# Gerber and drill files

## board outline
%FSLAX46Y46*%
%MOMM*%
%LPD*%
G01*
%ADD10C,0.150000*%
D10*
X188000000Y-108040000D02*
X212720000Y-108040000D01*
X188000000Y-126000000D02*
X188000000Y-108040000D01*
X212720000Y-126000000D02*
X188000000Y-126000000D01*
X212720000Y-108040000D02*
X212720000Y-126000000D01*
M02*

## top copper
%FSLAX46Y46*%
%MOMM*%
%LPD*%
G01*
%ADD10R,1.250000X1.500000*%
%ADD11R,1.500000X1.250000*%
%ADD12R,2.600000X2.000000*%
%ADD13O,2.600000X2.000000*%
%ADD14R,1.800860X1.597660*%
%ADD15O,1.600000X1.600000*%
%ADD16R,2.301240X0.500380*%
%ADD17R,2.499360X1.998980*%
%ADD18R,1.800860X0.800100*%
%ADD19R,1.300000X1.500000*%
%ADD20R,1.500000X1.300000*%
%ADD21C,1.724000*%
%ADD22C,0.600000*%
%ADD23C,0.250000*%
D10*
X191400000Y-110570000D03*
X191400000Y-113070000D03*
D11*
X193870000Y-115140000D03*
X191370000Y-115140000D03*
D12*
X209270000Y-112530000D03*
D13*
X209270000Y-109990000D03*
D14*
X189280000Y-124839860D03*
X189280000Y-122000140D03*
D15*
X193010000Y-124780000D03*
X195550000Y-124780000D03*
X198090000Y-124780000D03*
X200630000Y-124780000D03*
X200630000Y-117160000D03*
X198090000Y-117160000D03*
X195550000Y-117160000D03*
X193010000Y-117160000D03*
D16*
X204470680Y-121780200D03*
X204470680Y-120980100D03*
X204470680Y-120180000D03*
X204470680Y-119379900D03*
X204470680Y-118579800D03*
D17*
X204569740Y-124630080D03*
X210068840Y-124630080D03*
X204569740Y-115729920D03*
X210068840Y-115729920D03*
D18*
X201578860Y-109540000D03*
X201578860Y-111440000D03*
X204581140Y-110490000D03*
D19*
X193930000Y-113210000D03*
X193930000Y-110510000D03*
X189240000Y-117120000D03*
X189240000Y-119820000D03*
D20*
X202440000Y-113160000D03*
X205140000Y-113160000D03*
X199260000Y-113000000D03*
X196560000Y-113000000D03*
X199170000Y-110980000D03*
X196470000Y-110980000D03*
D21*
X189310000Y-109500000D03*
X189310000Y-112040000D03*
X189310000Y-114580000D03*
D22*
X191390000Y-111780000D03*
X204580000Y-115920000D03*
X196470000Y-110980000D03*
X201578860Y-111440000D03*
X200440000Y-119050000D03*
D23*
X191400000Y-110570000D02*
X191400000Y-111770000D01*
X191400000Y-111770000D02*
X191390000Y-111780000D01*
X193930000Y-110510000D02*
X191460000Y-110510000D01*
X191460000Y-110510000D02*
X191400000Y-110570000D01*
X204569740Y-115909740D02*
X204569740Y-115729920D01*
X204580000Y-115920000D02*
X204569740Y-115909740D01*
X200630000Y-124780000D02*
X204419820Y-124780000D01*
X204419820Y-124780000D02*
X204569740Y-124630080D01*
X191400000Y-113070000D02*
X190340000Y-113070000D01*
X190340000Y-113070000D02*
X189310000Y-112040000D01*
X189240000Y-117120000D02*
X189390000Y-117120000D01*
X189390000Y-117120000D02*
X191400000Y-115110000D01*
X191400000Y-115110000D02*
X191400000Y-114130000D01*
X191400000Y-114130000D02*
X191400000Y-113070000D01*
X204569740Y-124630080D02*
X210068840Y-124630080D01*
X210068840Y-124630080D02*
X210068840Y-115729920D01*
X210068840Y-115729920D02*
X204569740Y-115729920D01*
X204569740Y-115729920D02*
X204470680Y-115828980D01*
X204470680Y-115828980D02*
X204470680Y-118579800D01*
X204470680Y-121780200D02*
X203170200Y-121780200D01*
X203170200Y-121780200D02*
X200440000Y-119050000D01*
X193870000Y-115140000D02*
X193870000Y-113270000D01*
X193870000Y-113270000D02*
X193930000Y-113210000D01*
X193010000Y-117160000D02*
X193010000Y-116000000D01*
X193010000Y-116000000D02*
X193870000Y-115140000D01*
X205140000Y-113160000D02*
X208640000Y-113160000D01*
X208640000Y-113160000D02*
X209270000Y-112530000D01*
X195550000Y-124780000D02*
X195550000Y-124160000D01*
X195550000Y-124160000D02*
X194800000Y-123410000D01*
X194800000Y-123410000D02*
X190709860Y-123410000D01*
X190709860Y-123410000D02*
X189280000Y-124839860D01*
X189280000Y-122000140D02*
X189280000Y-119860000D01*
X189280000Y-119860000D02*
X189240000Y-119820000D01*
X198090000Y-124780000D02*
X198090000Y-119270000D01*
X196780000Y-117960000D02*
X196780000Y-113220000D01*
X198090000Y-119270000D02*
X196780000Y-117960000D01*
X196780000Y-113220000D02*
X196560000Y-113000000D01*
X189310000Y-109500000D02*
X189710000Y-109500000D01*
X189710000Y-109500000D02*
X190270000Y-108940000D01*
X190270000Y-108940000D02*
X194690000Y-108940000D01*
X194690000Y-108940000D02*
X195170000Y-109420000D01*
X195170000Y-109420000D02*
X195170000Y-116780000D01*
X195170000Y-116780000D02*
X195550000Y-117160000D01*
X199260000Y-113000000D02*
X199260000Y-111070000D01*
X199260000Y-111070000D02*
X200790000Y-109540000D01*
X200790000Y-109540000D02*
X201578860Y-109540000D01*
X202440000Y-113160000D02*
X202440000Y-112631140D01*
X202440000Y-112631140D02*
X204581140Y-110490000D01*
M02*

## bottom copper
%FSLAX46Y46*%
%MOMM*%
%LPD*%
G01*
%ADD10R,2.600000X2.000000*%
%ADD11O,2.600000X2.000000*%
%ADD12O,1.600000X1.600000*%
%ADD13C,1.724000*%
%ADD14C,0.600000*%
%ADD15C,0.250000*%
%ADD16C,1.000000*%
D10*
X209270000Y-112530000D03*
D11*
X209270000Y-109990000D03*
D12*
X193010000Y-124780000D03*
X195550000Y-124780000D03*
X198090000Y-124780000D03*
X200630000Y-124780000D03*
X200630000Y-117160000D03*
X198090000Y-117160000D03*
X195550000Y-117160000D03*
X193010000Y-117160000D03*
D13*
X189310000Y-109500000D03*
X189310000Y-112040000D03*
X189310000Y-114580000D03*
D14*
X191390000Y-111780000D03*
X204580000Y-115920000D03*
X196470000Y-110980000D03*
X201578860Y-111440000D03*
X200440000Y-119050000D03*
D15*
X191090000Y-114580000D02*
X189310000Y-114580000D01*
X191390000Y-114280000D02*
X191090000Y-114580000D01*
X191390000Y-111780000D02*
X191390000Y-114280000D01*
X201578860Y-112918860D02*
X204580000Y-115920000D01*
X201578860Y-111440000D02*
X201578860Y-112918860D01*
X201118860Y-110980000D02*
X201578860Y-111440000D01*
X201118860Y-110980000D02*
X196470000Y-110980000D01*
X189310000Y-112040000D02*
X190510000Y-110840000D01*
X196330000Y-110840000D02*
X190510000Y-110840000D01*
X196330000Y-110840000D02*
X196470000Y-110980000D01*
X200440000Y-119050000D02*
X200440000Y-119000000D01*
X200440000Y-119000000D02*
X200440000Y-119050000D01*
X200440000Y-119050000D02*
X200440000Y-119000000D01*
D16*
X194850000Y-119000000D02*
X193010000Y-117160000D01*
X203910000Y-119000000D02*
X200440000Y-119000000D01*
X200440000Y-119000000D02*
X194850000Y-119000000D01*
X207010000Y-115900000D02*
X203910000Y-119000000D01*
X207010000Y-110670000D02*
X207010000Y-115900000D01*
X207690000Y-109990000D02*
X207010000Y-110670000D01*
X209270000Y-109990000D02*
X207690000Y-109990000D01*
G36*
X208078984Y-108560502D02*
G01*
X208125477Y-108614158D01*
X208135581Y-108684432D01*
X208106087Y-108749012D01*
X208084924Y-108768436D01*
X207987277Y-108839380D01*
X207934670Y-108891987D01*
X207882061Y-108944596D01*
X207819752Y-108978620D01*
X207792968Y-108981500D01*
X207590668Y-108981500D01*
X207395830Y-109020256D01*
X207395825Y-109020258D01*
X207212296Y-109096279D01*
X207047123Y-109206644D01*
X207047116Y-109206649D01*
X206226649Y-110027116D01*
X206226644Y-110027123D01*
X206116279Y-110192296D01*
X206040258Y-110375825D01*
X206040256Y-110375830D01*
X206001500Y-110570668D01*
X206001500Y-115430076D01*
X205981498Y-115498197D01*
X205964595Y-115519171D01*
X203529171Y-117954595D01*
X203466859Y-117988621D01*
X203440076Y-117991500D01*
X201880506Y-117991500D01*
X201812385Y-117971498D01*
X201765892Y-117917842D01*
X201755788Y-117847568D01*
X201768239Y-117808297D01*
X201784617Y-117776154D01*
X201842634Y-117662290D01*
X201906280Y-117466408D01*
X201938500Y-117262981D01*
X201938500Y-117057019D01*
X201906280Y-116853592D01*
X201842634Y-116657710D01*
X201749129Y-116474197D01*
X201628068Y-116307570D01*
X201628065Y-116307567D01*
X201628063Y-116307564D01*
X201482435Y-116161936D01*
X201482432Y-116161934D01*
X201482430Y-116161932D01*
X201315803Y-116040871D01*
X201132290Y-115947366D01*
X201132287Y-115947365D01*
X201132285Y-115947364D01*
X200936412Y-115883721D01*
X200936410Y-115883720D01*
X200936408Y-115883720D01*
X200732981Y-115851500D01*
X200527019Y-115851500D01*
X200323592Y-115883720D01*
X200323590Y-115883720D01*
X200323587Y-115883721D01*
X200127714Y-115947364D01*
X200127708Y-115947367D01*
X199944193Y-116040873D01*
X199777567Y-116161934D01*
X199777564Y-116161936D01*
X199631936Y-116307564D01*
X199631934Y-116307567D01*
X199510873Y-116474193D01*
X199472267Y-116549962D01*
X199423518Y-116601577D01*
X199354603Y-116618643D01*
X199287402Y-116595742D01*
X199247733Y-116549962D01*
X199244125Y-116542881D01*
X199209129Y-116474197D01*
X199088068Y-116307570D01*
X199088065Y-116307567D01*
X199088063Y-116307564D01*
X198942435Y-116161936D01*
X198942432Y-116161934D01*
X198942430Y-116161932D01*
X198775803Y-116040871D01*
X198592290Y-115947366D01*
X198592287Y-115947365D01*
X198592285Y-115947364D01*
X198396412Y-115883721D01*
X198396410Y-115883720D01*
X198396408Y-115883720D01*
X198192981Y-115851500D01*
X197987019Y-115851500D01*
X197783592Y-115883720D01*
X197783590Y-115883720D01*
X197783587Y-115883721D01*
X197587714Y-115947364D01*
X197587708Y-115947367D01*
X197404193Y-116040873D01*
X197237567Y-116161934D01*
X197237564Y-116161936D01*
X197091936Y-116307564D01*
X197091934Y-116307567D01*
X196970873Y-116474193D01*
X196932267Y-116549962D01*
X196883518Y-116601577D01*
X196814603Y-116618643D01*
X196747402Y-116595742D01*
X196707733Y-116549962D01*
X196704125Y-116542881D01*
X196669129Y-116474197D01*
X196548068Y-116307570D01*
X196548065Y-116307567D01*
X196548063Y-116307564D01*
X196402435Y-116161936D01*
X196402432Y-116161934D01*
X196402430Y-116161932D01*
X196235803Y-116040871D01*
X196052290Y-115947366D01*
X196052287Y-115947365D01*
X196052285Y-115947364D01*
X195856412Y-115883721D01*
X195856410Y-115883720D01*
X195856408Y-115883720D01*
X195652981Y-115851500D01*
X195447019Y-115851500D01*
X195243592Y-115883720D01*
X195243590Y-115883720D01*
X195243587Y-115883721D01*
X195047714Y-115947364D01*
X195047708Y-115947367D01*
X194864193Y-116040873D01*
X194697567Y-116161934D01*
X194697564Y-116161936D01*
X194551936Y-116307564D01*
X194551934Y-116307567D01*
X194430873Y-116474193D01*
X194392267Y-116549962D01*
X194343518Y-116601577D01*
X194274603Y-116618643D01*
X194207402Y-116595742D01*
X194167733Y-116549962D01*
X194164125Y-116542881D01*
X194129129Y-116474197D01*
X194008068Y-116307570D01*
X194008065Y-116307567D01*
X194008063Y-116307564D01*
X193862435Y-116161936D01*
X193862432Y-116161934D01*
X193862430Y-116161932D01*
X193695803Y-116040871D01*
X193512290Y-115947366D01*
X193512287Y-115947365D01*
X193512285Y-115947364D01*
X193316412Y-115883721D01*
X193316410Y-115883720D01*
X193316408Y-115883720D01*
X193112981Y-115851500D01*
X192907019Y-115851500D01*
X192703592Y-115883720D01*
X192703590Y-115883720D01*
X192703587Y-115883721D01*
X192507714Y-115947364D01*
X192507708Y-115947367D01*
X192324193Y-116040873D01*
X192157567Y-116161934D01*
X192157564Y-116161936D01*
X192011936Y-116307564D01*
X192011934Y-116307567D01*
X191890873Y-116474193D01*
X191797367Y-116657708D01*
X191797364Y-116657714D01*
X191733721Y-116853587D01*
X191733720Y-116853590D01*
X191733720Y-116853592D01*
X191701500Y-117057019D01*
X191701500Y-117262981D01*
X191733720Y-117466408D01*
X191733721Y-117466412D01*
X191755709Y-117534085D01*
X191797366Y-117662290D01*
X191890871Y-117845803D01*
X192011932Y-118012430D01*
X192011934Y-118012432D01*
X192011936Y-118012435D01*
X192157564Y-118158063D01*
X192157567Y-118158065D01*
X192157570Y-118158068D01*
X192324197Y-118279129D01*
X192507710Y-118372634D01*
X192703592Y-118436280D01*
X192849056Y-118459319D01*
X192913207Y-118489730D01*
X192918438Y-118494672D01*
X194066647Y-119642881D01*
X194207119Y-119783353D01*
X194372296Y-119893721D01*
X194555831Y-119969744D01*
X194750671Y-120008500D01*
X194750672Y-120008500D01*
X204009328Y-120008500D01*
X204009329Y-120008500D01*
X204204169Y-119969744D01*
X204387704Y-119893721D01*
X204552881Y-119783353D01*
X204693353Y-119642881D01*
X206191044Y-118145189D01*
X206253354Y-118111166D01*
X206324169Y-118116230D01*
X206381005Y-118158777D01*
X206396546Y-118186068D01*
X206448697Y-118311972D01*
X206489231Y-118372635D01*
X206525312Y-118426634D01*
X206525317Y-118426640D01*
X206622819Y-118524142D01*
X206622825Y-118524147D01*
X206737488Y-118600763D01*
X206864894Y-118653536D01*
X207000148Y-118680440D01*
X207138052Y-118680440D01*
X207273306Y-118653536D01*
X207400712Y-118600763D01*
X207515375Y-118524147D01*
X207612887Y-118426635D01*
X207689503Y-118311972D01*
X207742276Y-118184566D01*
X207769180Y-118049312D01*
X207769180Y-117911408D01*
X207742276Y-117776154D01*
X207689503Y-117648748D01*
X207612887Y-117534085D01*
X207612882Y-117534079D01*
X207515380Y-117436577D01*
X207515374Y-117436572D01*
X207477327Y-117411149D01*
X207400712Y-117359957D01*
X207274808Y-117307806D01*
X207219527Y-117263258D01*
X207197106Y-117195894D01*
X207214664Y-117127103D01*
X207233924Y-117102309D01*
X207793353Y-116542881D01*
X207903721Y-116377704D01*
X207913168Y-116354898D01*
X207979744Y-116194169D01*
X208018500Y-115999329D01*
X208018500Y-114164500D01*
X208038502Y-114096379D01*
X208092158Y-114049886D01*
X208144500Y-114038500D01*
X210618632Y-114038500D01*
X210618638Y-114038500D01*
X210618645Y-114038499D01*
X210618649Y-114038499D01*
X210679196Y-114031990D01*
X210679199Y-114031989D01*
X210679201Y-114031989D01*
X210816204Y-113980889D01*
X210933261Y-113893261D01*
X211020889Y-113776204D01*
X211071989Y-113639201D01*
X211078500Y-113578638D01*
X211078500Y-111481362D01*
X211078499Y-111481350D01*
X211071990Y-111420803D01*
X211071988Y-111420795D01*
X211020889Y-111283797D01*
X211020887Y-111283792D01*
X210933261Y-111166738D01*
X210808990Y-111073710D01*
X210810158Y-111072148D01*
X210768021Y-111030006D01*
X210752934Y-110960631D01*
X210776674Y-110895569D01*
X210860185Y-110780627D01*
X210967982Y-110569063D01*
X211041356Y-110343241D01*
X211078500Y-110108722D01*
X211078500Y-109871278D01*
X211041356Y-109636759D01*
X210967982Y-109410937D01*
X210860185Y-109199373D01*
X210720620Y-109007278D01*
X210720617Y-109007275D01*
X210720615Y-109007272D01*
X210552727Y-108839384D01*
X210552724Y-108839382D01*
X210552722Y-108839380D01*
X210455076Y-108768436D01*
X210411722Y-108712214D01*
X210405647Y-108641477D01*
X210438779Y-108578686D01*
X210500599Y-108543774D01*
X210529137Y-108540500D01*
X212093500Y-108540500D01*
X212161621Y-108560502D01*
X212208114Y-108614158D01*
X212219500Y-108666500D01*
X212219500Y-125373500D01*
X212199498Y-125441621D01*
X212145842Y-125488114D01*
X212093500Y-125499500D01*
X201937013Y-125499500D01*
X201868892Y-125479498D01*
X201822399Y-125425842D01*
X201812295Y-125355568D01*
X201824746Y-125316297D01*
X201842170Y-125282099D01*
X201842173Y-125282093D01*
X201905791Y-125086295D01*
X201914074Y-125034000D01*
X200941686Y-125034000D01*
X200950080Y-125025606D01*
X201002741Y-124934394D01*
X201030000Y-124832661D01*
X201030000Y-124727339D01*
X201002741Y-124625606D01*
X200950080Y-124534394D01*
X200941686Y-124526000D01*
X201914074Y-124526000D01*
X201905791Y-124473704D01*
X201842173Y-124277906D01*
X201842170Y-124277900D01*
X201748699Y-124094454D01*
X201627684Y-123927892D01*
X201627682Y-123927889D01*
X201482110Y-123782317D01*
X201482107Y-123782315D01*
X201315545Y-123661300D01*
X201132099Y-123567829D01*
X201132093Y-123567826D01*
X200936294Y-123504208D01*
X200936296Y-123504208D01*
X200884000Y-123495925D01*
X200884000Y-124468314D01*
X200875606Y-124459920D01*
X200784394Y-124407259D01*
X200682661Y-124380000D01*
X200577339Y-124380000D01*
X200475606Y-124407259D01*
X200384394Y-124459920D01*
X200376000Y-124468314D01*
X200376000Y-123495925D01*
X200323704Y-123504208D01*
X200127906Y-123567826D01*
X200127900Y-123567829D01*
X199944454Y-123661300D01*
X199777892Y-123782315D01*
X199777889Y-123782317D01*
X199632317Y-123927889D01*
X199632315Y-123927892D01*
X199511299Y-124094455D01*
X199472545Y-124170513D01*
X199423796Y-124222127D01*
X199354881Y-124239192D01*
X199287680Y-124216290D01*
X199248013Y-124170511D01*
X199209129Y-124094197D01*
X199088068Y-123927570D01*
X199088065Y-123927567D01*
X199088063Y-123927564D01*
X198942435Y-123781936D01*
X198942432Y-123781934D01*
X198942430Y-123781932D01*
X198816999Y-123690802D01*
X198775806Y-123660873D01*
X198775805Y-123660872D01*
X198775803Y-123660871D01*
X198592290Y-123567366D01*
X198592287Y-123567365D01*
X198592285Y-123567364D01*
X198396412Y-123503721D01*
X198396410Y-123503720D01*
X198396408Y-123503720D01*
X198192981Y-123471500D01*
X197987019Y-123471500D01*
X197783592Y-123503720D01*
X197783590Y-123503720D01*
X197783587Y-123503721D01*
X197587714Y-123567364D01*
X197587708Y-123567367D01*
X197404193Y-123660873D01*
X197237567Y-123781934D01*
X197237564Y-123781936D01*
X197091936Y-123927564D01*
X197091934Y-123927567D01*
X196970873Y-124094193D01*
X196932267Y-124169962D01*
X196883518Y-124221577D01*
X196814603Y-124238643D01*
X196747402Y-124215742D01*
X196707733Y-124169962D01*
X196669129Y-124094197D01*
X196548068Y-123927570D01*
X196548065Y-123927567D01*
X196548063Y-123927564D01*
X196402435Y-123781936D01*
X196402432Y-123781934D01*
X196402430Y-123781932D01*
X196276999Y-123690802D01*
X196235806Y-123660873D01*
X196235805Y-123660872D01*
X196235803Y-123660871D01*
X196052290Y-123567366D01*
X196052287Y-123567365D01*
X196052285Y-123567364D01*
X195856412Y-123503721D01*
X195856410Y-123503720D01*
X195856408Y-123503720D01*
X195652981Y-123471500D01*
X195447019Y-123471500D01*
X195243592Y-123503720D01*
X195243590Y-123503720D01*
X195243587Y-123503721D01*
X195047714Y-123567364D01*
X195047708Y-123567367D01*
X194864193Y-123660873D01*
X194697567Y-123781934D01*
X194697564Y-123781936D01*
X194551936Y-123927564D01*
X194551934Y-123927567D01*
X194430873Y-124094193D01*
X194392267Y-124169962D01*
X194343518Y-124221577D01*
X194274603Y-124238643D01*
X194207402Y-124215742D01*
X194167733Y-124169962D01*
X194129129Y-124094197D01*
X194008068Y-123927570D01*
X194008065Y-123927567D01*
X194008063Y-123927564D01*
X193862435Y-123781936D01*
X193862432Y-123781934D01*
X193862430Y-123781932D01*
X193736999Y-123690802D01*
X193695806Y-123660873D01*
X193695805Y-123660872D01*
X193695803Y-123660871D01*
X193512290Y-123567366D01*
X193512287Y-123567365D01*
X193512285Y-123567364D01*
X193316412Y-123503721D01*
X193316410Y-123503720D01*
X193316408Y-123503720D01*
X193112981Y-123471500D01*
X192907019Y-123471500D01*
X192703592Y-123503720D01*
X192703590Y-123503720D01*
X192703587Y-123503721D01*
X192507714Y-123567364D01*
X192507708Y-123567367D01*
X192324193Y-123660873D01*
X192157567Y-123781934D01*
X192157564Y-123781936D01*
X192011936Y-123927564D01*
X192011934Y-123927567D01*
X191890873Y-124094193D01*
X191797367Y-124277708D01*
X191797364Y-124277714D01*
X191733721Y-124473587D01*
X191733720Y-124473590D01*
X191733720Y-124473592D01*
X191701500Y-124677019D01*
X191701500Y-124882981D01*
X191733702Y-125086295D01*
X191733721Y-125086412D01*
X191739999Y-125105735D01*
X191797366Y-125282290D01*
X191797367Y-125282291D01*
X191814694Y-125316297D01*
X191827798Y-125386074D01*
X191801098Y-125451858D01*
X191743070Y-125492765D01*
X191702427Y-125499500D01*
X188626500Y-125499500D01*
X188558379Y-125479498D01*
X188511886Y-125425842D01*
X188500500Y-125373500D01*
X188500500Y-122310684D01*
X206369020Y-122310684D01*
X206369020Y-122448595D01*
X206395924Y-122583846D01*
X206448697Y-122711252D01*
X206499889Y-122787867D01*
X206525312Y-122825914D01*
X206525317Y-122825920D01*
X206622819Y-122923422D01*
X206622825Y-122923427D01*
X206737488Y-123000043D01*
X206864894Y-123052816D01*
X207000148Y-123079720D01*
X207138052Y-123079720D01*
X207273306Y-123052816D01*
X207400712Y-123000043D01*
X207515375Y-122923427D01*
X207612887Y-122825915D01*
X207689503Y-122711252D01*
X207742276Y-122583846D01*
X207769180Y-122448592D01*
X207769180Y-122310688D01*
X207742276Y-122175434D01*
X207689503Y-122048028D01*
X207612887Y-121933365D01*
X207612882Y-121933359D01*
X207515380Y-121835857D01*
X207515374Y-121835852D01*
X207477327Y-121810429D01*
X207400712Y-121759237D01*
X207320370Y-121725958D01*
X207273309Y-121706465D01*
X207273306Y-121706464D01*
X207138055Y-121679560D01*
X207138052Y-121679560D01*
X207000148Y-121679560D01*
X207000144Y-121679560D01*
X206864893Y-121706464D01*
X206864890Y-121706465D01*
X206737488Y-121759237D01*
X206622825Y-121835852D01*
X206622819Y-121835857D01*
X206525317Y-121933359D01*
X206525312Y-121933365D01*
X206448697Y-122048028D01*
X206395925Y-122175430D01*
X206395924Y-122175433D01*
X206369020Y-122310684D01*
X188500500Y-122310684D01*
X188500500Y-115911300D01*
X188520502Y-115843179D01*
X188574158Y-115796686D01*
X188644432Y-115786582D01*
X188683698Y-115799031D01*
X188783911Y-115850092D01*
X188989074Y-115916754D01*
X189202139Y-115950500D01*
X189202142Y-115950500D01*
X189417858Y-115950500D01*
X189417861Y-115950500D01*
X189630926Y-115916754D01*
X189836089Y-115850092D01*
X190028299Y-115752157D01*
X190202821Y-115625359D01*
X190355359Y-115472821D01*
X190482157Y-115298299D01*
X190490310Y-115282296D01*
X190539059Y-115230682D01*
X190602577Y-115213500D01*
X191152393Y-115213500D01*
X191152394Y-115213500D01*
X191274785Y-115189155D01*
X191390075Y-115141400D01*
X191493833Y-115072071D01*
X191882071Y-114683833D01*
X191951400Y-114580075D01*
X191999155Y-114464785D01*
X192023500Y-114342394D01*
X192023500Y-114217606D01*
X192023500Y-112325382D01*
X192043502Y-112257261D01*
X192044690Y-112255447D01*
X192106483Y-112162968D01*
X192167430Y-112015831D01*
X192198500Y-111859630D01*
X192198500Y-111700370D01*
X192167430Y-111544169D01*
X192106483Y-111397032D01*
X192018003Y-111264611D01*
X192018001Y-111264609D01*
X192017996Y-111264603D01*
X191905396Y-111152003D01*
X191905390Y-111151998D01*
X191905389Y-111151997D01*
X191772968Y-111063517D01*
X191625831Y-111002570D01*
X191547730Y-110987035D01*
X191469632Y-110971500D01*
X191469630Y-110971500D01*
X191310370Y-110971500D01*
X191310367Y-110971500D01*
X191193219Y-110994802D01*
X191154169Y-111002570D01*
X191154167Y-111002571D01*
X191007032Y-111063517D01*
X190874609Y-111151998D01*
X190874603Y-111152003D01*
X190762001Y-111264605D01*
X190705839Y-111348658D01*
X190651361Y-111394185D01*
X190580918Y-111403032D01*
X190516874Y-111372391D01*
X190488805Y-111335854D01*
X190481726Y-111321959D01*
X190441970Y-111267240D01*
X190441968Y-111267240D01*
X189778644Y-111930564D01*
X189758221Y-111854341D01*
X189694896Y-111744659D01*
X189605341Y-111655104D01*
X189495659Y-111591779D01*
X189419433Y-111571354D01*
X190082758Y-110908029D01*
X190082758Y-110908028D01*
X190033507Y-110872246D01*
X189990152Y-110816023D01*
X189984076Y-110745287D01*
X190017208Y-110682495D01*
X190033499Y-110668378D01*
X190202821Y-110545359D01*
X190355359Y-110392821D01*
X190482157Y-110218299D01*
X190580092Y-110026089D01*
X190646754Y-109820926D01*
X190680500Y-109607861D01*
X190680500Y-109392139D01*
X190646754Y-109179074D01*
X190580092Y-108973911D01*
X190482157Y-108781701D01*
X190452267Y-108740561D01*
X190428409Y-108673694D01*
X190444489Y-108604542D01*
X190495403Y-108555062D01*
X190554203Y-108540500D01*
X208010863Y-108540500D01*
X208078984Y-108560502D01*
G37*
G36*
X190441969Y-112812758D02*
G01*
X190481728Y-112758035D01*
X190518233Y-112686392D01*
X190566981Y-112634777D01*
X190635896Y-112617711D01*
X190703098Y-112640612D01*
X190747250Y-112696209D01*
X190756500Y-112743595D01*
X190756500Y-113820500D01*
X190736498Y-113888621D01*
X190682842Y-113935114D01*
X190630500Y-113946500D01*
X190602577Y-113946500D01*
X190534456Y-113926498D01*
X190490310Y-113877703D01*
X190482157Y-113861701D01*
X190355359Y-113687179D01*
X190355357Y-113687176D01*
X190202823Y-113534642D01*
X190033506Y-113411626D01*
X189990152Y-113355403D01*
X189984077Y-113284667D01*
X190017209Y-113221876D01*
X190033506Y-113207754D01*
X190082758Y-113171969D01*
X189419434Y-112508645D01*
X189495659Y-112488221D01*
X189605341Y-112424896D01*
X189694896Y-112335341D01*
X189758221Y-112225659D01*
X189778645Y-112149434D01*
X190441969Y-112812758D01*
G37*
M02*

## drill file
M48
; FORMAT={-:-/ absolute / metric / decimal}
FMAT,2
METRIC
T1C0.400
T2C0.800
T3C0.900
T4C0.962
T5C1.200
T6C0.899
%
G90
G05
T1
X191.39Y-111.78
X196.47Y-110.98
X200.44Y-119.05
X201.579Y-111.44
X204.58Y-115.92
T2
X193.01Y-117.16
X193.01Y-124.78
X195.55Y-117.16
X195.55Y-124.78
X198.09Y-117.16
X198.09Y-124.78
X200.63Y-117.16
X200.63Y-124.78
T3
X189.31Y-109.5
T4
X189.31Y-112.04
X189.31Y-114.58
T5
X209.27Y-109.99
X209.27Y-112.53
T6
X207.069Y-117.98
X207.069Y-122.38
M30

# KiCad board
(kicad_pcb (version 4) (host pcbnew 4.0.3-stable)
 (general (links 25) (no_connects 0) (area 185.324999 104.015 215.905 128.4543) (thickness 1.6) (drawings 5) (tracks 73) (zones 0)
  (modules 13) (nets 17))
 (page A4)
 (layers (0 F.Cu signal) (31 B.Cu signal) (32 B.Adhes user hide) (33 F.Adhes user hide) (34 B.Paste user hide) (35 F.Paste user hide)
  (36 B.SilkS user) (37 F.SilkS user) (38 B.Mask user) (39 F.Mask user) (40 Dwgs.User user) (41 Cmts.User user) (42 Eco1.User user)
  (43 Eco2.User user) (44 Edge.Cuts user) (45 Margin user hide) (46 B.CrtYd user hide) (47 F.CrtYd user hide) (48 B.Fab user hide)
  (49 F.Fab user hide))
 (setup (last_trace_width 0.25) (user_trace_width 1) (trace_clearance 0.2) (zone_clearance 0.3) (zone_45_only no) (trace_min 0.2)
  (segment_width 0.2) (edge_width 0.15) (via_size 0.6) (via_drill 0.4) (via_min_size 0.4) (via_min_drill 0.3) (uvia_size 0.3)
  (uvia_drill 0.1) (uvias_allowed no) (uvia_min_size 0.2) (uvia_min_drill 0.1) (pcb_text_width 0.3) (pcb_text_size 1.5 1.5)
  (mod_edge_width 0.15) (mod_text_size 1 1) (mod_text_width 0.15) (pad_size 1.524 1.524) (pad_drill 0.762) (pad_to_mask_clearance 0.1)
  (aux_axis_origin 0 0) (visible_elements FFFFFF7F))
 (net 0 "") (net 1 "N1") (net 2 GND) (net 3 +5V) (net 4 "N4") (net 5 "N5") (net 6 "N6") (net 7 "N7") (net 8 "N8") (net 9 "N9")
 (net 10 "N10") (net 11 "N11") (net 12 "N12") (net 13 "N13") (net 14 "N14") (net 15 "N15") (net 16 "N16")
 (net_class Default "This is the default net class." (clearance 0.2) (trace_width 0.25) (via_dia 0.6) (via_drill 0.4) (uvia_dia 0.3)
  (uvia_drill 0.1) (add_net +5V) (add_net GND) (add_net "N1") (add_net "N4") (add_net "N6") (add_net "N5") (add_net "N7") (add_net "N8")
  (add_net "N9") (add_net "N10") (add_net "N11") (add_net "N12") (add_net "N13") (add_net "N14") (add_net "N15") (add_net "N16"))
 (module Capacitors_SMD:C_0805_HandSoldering (layer F.Cu) (at 191.4 111.82 270)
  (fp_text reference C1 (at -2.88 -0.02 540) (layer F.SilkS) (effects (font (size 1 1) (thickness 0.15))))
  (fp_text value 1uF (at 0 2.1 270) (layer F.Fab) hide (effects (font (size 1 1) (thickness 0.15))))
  (pad 1 smd rect (at -1.25 0 270) (size 1.5 1.25) (layers F.Cu F.Paste F.Mask) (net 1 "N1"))
  (pad 2 smd rect (at 1.25 0 270) (size 1.5 1.25) (layers F.Cu F.Paste F.Mask) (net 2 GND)))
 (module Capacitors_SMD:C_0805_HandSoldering (layer F.Cu) (at 192.62 115.14 180)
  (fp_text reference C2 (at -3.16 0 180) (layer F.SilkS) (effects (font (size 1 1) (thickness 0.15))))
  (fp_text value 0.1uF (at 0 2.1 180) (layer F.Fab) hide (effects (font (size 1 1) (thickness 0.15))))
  (pad 1 smd rect (at -1.25 0 180) (size 1.5 1.25) (layers F.Cu F.Paste F.Mask) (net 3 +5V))
  (pad 2 smd rect (at 1.25 0 180) (size 1.5 1.25) (layers F.Cu F.Paste F.Mask) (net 2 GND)))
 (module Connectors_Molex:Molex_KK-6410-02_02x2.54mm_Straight (layer F.Cu) (at 209.27 112.53 90)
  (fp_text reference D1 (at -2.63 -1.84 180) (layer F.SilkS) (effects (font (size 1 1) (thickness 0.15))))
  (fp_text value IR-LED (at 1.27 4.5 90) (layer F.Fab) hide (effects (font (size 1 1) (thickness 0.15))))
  (pad 1 thru_hole rect (at 0 0 90) (size 2 2.6) (drill 1.2) (layers *.Cu *.Mask F.SilkS) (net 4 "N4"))
  (pad 2 thru_hole oval (at 2.54 0 90) (size 2 2.6) (drill 1.2) (layers *.Cu *.Mask F.SilkS) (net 3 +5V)))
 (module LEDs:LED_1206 (layer F.Cu) (at 189.28 123.42 270)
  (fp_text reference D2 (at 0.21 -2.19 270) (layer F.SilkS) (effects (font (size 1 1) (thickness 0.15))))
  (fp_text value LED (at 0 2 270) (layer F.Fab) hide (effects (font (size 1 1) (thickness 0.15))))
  (pad 2 smd rect (at 1.41986 0 90) (size 1.59766 1.80086) (layers F.Cu F.Paste F.Mask) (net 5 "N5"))
  (pad 1 smd rect (at -1.41986 0 90) (size 1.59766 1.80086) (layers F.Cu F.Paste F.Mask) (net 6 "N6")))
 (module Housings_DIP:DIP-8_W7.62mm (layer F.Cu) (at 193.01 124.78 90)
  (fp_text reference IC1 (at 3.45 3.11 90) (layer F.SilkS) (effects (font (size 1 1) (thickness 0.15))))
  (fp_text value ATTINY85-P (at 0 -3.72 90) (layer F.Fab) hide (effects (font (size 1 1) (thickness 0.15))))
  (pad 1 thru_hole oval (at 0 0 90) (size 1.6 1.6) (drill 0.8) (layers *.Cu *.Mask F.SilkS) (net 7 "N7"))
  (pad 2 thru_hole oval (at 0 2.54 90) (size 1.6 1.6) (drill 0.8) (layers *.Cu *.Mask F.SilkS) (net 5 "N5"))
  (pad 3 thru_hole oval (at 0 5.08 90) (size 1.6 1.6) (drill 0.8) (layers *.Cu *.Mask F.SilkS) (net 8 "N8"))
  (pad 4 thru_hole oval (at 0 7.62 90) (size 1.6 1.6) (drill 0.8) (layers *.Cu *.Mask F.SilkS) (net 2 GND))
  (pad 5 thru_hole oval (at 7.62 7.62 90) (size 1.6 1.6) (drill 0.8) (layers *.Cu *.Mask F.SilkS) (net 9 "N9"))
  (pad 6 thru_hole oval (at 7.62 5.08 90) (size 1.6 1.6) (drill 0.8) (layers *.Cu *.Mask F.SilkS) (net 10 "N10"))
  (pad 7 thru_hole oval (at 7.62 2.54 90) (size 1.6 1.6) (drill 0.8) (layers *.Cu *.Mask F.SilkS) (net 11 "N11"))
  (pad 8 thru_hole oval (at 7.62 0 90) (size 1.6 1.6) (drill 0.8) (layers *.Cu *.Mask F.SilkS) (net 3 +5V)))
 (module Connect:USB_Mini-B (layer F.Cu) (at 207.92 120.18 180)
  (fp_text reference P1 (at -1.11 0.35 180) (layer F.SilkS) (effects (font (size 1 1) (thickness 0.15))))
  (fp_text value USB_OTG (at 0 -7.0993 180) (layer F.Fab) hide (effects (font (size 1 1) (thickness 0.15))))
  (pad 1 smd rect (at 3.44932 -1.6002 180) (size 2.30124 0.50038) (layers F.Cu F.Paste F.Mask) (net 3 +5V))
  (pad 2 smd rect (at 3.44932 -0.8001 180) (size 2.30124 0.50038) (layers F.Cu F.Paste F.Mask) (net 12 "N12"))
  (pad 3 smd rect (at 3.44932 0 180) (size 2.30124 0.50038) (layers F.Cu F.Paste F.Mask) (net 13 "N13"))
  (pad 4 smd rect (at 3.44932 0.8001 180) (size 2.30124 0.50038) (layers F.Cu F.Paste F.Mask) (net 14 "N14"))
  (pad 5 smd rect (at 3.44932 1.6002 180) (size 2.30124 0.50038) (layers F.Cu F.Paste F.Mask) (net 2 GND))
  (pad 6 smd rect (at 3.35026 -4.45008 180) (size 2.49936 1.99898) (layers F.Cu F.Paste F.Mask) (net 2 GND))
  (pad 6 smd rect (at -2.14884 -4.45008 180) (size 2.49936 1.99898) (layers F.Cu F.Paste F.Mask) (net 2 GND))
  (pad 6 smd rect (at 3.35026 4.45008 180) (size 2.49936 1.99898) (layers F.Cu F.Paste F.Mask) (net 2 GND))
  (pad 6 smd rect (at -2.14884 4.45008 180) (size 2.49936 1.99898) (layers F.Cu F.Paste F.Mask) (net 2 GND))
  (pad "" np_thru_hole circle (at 0.8509 -2.19964 180) (size 0.89916 0.89916) (drill 0.89916) (layers *.Cu *.Mask F.SilkS))
  (pad "" np_thru_hole circle (at 0.8509 2.19964 180) (size 0.89916 0.89916) (drill 0.89916) (layers *.Cu *.Mask F.SilkS)))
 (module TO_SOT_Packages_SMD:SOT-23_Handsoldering (layer F.Cu) (at 203.08 110.49 270)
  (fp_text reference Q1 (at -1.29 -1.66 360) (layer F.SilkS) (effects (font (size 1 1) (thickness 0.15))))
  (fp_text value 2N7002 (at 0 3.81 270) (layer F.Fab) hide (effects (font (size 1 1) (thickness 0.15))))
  (pad 1 smd rect (at -0.95 1.50114 270) (size 0.8001 1.80086) (layers F.Cu F.Paste F.Mask) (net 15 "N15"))
  (pad 2 smd rect (at 0.95 1.50114 270) (size 0.8001 1.80086) (layers F.Cu F.Paste F.Mask) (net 2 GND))
  (pad 3 smd rect (at 0 -1.50114 270) (size 0.8001 1.80086) (layers F.Cu F.Paste F.Mask) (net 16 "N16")))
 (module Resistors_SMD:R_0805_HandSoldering (layer F.Cu) (at 193.93 111.86 90)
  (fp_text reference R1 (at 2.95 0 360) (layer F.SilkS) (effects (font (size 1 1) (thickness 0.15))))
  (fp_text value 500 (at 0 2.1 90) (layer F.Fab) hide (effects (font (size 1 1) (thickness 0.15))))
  (pad 1 smd rect (at -1.35 0 90) (size 1.5 1.3) (layers F.Cu F.Paste F.Mask) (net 3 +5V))
  (pad 2 smd rect (at 1.35 0 90) (size 1.5 1.3) (layers F.Cu F.Paste F.Mask) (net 1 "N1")))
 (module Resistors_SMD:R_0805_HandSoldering (layer F.Cu) (at 189.24 118.47 270)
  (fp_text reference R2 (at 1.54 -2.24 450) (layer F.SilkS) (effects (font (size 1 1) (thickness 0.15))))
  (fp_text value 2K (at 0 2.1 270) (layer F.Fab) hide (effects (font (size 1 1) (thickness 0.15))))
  (pad 1 smd rect (at -1.35 0 270) (size 1.5 1.3) (layers F.Cu F.Paste F.Mask) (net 2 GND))
  (pad 2 smd rect (at 1.35 0 270) (size 1.5 1.3) (layers F.Cu F.Paste F.Mask) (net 6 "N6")))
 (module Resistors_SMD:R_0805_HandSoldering (layer F.Cu) (at 203.79 113.16)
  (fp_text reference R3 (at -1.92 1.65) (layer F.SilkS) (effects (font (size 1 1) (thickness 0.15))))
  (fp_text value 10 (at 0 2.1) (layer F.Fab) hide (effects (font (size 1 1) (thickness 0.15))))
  (pad 1 smd rect (at -1.35 0) (size 1.5 1.3) (layers F.Cu F.Paste F.Mask) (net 16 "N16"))
  (pad 2 smd rect (at 1.35 0) (size 1.5 1.3) (layers F.Cu F.Paste F.Mask) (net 4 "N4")))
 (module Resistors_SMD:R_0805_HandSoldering (layer F.Cu) (at 197.91 113 180)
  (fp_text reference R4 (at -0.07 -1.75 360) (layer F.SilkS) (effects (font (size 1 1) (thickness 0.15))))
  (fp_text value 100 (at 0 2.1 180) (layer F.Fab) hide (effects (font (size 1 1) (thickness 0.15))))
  (pad 1 smd rect (at -1.35 0 180) (size 1.5 1.3) (layers F.Cu F.Paste F.Mask) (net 15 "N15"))
  (pad 2 smd rect (at 1.35 0 180) (size 1.5 1.3) (layers F.Cu F.Paste F.Mask) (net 8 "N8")))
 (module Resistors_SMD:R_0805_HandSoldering (layer F.Cu) (at 197.82 110.98 180)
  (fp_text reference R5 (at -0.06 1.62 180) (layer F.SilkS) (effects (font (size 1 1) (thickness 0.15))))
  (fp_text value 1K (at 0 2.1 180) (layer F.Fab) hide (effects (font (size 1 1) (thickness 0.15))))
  (pad 1 smd rect (at -1.35 0 180) (size 1.5 1.3) (layers F.Cu F.Paste F.Mask) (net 15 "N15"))
  (pad 2 smd rect (at 1.35 0 180) (size 1.5 1.3) (layers F.Cu F.Paste F.Mask) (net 2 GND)))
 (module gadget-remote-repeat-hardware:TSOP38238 (layer F.Cu) (at 187.86 112.04 270)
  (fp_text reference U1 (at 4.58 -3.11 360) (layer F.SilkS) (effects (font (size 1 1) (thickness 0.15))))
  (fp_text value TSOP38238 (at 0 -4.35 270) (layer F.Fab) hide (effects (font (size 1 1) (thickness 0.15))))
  (pad 1 thru_hole circle (at -2.54 -1.45 270) (size 1.724 1.724) (drill 0.9) (layers *.Cu *.Mask) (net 11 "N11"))
  (pad 2 thru_hole circle (at 0 -1.45 270) (size 1.724 1.724) (drill 0.962) (layers *.Cu *.Mask) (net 2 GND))
  (pad 3 thru_hole circle (at 2.54 -1.45 270) (size 1.724 1.724) (drill 0.962) (layers *.Cu *.Mask) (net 1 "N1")))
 (gr_line (start 188 108.04) (end 212.72 108.04) (angle 90) (layer Edge.Cuts) (width 0.15))
 (gr_line (start 188 126) (end 188 108.04) (angle 90) (layer Edge.Cuts) (width 0.15))
 (gr_line (start 212.72 126) (end 188 126) (angle 90) (layer Edge.Cuts) (width 0.15))
 (gr_line (start 212.72 108.04) (end 212.72 126) (angle 90) (layer Edge.Cuts) (width 0.15))
 (segment (start 191.4 110.57) (end 191.4 111.77) (width 0.25) (layer F.Cu) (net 1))
 (segment (start 191.09 114.58) (end 189.31 114.58) (width 0.25) (layer B.Cu) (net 1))
 (segment (start 191.39 114.28) (end 191.09 114.58) (width 0.25) (layer B.Cu) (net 1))
 (segment (start 191.39 111.78) (end 191.39 114.28) (width 0.25) (layer B.Cu) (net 1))
 (via (at 191.39 111.78) (size 0.6) (drill 0.4) (layers F.Cu B.Cu) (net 1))
 (segment (start 191.4 111.77) (end 191.39 111.78) (width 0.25) (layer F.Cu) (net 1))
 (segment (start 193.93 110.51) (end 191.46 110.51) (width 0.25) (layer F.Cu) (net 1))
 (segment (start 191.46 110.51) (end 191.4 110.57) (width 0.25) (layer F.Cu) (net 1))
 (segment (start 204.56974 115.90974) (end 204.56974 115.72992) (width 0.25) (layer F.Cu) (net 2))
 (segment (start 204.58 115.92) (end 204.56974 115.90974) (width 0.25) (layer F.Cu) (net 2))
 (via (at 204.58 115.92) (size 0.6) (drill 0.4) (layers F.Cu B.Cu) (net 2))
 (segment (start 201.57886 112.91886) (end 204.58 115.92) (width 0.25) (layer B.Cu) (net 2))
 (segment (start 201.57886 111.44) (end 201.57886 112.91886) (width 0.25) (layer B.Cu) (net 2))
 (segment (start 201.11886 110.98) (end 201.57886 111.44) (width 0.25) (layer B.Cu) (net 2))
 (segment (start 201.11886 110.98) (end 196.47 110.98) (width 0.25) (layer B.Cu) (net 2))
 (via (at 196.47 110.98) (size 0.6) (drill 0.4) (layers F.Cu B.Cu) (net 2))
 (segment (start 189.31 112.04) (end 190.51 110.84) (width 0.25) (layer B.Cu) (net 2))
 (segment (start 196.33 110.84) (end 190.51 110.84) (width 0.25) (layer B.Cu) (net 2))
 (segment (start 196.33 110.84) (end 196.47 110.98) (width 0.25) (layer B.Cu) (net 2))
 (via (at 201.57886 111.44) (size 0.6) (drill 0.4) (layers F.Cu B.Cu) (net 2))
 (segment (start 200.63 124.78) (end 204.41982 124.78) (width 0.25) (layer F.Cu) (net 2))
 (segment (start 204.41982 124.78) (end 204.56974 124.63008) (width 0.25) (layer F.Cu) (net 2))
 (segment (start 191.4 113.07) (end 190.34 113.07) (width 0.25) (layer F.Cu) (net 2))
 (segment (start 190.34 113.07) (end 189.31 112.04) (width 0.25) (layer F.Cu) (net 2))
 (segment (start 189.24 117.12) (end 189.39 117.12) (width 0.25) (layer F.Cu) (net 2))
 (segment (start 189.39 117.12) (end 191.4 115.11) (width 0.25) (layer F.Cu) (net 2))
 (segment (start 191.4 115.11) (end 191.4 114.13) (width 0.25) (layer F.Cu) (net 2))
 (segment (start 191.4 114.13) (end 191.4 113.07) (width 0.25) (layer F.Cu) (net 2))
 (segment (start 204.56974 124.63008) (end 210.06884 124.63008) (width 0.25) (layer F.Cu) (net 2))
 (segment (start 210.06884 124.63008) (end 210.06884 115.72992) (width 0.25) (layer F.Cu) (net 2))
 (segment (start 210.06884 115.72992) (end 204.56974 115.72992) (width 0.25) (layer F.Cu) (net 2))
 (segment (start 204.56974 115.72992) (end 204.47068 115.82898) (width 0.25) (layer F.Cu) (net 2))
 (segment (start 204.47068 115.82898) (end 204.47068 118.5798) (width 0.25) (layer F.Cu) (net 2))
 (segment (start 204.47068 121.7802) (end 203.1702 121.7802) (width 0.25) (layer F.Cu) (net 3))
 (via (at 200.44 119.05) (size 0.6) (drill 0.4) (layers F.Cu B.Cu) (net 3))
 (segment (start 203.1702 121.7802) (end 200.44 119.05) (width 0.25) (layer F.Cu) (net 3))
 (segment (start 200.44 119.05) (end 200.44 119) (width 0.25) (layer B.Cu) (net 3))
 (segment (start 200.44 119) (end 200.44 119.05) (width 0.25) (layer B.Cu) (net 3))
 (segment (start 200.44 119.05) (end 200.44 119) (width 0.25) (layer B.Cu) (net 3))
 (segment (start 194.85 119) (end 193.01 117.16) (width 1) (layer B.Cu) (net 3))
 (segment (start 203.91 119) (end 200.44 119) (width 1) (layer B.Cu) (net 3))
 (segment (start 200.44 119) (end 194.85 119) (width 1) (layer B.Cu) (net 3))
 (segment (start 207.01 115.9) (end 203.91 119) (width 1) (layer B.Cu) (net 3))
 (segment (start 207.01 110.67) (end 207.01 115.9) (width 1) (layer B.Cu) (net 3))
 (segment (start 207.69 109.99) (end 207.01 110.67) (width 1) (layer B.Cu) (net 3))
 (segment (start 209.27 109.99) (end 207.69 109.99) (width 1) (layer B.Cu) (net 3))
 (segment (start 193.87 115.14) (end 193.87 113.27) (width 0.25) (layer F.Cu) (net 3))
 (segment (start 193.87 113.27) (end 193.93 113.21) (width 0.25) (layer F.Cu) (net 3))
 (segment (start 193.01 117.16) (end 193.01 116) (width 0.25) (layer F.Cu) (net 3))
 (segment (start 193.01 116) (end 193.87 115.14) (width 0.25) (layer F.Cu) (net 3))
 (segment (start 205.14 113.16) (end 208.64 113.16) (width 0.25) (layer F.Cu) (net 4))
 (segment (start 208.64 113.16) (end 209.27 112.53) (width 0.25) (layer F.Cu) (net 4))
 (segment (start 195.55 124.78) (end 195.55 124.16) (width 0.25) (layer F.Cu) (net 5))
 (segment (start 195.55 124.16) (end 194.8 123.41) (width 0.25) (layer F.Cu) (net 5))
 (segment (start 194.8 123.41) (end 190.70986 123.41) (width 0.25) (layer F.Cu) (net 5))
 (segment (start 190.70986 123.41) (end 189.28 124.83986) (width 0.25) (layer F.Cu) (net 5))
 (segment (start 189.28 122.00014) (end 189.28 119.86) (width 0.25) (layer F.Cu) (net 6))
 (segment (start 189.28 119.86) (end 189.24 119.82) (width 0.25) (layer F.Cu) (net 6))
 (segment (start 198.09 124.78) (end 198.09 119.27) (width 0.25) (layer F.Cu) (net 8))
 (segment (start 196.78 117.96) (end 196.78 113.22) (width 0.25) (layer F.Cu) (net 8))
 (segment (start 198.09 119.27) (end 196.78 117.96) (width 0.25) (layer F.Cu) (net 8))
 (segment (start 196.78 113.22) (end 196.56 113) (width 0.25) (layer F.Cu) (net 8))
 (segment (start 189.31 109.5) (end 189.71 109.5) (width 0.25) (layer F.Cu) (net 11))
 (segment (start 189.71 109.5) (end 190.27 108.94) (width 0.25) (layer F.Cu) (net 11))
 (segment (start 190.27 108.94) (end 194.69 108.94) (width 0.25) (layer F.Cu) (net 11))
 (segment (start 194.69 108.94) (end 195.17 109.42) (width 0.25) (layer F.Cu) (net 11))
 (segment (start 195.17 109.42) (end 195.17 116.78) (width 0.25) (layer F.Cu) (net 11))
 (segment (start 195.17 116.78) (end 195.55 117.16) (width 0.25) (layer F.Cu) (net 11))
 (segment (start 199.26 113) (end 199.26 111.07) (width 0.25) (layer F.Cu) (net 15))
 (segment (start 199.26 111.07) (end 200.79 109.54) (width 0.25) (layer F.Cu) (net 15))
 (segment (start 200.79 109.54) (end 201.57886 109.54) (width 0.25) (layer F.Cu) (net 15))
 (segment (start 202.44 113.16) (end 202.44 112.63114) (width 0.25) (layer F.Cu) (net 16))
 (segment (start 202.44 112.63114) (end 204.58114 110.49) (width 0.25) (layer F.Cu) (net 16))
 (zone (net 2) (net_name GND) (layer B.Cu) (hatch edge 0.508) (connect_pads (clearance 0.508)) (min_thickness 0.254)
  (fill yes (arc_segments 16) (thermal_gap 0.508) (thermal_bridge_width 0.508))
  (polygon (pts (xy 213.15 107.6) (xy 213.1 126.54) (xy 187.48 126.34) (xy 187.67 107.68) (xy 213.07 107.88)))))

